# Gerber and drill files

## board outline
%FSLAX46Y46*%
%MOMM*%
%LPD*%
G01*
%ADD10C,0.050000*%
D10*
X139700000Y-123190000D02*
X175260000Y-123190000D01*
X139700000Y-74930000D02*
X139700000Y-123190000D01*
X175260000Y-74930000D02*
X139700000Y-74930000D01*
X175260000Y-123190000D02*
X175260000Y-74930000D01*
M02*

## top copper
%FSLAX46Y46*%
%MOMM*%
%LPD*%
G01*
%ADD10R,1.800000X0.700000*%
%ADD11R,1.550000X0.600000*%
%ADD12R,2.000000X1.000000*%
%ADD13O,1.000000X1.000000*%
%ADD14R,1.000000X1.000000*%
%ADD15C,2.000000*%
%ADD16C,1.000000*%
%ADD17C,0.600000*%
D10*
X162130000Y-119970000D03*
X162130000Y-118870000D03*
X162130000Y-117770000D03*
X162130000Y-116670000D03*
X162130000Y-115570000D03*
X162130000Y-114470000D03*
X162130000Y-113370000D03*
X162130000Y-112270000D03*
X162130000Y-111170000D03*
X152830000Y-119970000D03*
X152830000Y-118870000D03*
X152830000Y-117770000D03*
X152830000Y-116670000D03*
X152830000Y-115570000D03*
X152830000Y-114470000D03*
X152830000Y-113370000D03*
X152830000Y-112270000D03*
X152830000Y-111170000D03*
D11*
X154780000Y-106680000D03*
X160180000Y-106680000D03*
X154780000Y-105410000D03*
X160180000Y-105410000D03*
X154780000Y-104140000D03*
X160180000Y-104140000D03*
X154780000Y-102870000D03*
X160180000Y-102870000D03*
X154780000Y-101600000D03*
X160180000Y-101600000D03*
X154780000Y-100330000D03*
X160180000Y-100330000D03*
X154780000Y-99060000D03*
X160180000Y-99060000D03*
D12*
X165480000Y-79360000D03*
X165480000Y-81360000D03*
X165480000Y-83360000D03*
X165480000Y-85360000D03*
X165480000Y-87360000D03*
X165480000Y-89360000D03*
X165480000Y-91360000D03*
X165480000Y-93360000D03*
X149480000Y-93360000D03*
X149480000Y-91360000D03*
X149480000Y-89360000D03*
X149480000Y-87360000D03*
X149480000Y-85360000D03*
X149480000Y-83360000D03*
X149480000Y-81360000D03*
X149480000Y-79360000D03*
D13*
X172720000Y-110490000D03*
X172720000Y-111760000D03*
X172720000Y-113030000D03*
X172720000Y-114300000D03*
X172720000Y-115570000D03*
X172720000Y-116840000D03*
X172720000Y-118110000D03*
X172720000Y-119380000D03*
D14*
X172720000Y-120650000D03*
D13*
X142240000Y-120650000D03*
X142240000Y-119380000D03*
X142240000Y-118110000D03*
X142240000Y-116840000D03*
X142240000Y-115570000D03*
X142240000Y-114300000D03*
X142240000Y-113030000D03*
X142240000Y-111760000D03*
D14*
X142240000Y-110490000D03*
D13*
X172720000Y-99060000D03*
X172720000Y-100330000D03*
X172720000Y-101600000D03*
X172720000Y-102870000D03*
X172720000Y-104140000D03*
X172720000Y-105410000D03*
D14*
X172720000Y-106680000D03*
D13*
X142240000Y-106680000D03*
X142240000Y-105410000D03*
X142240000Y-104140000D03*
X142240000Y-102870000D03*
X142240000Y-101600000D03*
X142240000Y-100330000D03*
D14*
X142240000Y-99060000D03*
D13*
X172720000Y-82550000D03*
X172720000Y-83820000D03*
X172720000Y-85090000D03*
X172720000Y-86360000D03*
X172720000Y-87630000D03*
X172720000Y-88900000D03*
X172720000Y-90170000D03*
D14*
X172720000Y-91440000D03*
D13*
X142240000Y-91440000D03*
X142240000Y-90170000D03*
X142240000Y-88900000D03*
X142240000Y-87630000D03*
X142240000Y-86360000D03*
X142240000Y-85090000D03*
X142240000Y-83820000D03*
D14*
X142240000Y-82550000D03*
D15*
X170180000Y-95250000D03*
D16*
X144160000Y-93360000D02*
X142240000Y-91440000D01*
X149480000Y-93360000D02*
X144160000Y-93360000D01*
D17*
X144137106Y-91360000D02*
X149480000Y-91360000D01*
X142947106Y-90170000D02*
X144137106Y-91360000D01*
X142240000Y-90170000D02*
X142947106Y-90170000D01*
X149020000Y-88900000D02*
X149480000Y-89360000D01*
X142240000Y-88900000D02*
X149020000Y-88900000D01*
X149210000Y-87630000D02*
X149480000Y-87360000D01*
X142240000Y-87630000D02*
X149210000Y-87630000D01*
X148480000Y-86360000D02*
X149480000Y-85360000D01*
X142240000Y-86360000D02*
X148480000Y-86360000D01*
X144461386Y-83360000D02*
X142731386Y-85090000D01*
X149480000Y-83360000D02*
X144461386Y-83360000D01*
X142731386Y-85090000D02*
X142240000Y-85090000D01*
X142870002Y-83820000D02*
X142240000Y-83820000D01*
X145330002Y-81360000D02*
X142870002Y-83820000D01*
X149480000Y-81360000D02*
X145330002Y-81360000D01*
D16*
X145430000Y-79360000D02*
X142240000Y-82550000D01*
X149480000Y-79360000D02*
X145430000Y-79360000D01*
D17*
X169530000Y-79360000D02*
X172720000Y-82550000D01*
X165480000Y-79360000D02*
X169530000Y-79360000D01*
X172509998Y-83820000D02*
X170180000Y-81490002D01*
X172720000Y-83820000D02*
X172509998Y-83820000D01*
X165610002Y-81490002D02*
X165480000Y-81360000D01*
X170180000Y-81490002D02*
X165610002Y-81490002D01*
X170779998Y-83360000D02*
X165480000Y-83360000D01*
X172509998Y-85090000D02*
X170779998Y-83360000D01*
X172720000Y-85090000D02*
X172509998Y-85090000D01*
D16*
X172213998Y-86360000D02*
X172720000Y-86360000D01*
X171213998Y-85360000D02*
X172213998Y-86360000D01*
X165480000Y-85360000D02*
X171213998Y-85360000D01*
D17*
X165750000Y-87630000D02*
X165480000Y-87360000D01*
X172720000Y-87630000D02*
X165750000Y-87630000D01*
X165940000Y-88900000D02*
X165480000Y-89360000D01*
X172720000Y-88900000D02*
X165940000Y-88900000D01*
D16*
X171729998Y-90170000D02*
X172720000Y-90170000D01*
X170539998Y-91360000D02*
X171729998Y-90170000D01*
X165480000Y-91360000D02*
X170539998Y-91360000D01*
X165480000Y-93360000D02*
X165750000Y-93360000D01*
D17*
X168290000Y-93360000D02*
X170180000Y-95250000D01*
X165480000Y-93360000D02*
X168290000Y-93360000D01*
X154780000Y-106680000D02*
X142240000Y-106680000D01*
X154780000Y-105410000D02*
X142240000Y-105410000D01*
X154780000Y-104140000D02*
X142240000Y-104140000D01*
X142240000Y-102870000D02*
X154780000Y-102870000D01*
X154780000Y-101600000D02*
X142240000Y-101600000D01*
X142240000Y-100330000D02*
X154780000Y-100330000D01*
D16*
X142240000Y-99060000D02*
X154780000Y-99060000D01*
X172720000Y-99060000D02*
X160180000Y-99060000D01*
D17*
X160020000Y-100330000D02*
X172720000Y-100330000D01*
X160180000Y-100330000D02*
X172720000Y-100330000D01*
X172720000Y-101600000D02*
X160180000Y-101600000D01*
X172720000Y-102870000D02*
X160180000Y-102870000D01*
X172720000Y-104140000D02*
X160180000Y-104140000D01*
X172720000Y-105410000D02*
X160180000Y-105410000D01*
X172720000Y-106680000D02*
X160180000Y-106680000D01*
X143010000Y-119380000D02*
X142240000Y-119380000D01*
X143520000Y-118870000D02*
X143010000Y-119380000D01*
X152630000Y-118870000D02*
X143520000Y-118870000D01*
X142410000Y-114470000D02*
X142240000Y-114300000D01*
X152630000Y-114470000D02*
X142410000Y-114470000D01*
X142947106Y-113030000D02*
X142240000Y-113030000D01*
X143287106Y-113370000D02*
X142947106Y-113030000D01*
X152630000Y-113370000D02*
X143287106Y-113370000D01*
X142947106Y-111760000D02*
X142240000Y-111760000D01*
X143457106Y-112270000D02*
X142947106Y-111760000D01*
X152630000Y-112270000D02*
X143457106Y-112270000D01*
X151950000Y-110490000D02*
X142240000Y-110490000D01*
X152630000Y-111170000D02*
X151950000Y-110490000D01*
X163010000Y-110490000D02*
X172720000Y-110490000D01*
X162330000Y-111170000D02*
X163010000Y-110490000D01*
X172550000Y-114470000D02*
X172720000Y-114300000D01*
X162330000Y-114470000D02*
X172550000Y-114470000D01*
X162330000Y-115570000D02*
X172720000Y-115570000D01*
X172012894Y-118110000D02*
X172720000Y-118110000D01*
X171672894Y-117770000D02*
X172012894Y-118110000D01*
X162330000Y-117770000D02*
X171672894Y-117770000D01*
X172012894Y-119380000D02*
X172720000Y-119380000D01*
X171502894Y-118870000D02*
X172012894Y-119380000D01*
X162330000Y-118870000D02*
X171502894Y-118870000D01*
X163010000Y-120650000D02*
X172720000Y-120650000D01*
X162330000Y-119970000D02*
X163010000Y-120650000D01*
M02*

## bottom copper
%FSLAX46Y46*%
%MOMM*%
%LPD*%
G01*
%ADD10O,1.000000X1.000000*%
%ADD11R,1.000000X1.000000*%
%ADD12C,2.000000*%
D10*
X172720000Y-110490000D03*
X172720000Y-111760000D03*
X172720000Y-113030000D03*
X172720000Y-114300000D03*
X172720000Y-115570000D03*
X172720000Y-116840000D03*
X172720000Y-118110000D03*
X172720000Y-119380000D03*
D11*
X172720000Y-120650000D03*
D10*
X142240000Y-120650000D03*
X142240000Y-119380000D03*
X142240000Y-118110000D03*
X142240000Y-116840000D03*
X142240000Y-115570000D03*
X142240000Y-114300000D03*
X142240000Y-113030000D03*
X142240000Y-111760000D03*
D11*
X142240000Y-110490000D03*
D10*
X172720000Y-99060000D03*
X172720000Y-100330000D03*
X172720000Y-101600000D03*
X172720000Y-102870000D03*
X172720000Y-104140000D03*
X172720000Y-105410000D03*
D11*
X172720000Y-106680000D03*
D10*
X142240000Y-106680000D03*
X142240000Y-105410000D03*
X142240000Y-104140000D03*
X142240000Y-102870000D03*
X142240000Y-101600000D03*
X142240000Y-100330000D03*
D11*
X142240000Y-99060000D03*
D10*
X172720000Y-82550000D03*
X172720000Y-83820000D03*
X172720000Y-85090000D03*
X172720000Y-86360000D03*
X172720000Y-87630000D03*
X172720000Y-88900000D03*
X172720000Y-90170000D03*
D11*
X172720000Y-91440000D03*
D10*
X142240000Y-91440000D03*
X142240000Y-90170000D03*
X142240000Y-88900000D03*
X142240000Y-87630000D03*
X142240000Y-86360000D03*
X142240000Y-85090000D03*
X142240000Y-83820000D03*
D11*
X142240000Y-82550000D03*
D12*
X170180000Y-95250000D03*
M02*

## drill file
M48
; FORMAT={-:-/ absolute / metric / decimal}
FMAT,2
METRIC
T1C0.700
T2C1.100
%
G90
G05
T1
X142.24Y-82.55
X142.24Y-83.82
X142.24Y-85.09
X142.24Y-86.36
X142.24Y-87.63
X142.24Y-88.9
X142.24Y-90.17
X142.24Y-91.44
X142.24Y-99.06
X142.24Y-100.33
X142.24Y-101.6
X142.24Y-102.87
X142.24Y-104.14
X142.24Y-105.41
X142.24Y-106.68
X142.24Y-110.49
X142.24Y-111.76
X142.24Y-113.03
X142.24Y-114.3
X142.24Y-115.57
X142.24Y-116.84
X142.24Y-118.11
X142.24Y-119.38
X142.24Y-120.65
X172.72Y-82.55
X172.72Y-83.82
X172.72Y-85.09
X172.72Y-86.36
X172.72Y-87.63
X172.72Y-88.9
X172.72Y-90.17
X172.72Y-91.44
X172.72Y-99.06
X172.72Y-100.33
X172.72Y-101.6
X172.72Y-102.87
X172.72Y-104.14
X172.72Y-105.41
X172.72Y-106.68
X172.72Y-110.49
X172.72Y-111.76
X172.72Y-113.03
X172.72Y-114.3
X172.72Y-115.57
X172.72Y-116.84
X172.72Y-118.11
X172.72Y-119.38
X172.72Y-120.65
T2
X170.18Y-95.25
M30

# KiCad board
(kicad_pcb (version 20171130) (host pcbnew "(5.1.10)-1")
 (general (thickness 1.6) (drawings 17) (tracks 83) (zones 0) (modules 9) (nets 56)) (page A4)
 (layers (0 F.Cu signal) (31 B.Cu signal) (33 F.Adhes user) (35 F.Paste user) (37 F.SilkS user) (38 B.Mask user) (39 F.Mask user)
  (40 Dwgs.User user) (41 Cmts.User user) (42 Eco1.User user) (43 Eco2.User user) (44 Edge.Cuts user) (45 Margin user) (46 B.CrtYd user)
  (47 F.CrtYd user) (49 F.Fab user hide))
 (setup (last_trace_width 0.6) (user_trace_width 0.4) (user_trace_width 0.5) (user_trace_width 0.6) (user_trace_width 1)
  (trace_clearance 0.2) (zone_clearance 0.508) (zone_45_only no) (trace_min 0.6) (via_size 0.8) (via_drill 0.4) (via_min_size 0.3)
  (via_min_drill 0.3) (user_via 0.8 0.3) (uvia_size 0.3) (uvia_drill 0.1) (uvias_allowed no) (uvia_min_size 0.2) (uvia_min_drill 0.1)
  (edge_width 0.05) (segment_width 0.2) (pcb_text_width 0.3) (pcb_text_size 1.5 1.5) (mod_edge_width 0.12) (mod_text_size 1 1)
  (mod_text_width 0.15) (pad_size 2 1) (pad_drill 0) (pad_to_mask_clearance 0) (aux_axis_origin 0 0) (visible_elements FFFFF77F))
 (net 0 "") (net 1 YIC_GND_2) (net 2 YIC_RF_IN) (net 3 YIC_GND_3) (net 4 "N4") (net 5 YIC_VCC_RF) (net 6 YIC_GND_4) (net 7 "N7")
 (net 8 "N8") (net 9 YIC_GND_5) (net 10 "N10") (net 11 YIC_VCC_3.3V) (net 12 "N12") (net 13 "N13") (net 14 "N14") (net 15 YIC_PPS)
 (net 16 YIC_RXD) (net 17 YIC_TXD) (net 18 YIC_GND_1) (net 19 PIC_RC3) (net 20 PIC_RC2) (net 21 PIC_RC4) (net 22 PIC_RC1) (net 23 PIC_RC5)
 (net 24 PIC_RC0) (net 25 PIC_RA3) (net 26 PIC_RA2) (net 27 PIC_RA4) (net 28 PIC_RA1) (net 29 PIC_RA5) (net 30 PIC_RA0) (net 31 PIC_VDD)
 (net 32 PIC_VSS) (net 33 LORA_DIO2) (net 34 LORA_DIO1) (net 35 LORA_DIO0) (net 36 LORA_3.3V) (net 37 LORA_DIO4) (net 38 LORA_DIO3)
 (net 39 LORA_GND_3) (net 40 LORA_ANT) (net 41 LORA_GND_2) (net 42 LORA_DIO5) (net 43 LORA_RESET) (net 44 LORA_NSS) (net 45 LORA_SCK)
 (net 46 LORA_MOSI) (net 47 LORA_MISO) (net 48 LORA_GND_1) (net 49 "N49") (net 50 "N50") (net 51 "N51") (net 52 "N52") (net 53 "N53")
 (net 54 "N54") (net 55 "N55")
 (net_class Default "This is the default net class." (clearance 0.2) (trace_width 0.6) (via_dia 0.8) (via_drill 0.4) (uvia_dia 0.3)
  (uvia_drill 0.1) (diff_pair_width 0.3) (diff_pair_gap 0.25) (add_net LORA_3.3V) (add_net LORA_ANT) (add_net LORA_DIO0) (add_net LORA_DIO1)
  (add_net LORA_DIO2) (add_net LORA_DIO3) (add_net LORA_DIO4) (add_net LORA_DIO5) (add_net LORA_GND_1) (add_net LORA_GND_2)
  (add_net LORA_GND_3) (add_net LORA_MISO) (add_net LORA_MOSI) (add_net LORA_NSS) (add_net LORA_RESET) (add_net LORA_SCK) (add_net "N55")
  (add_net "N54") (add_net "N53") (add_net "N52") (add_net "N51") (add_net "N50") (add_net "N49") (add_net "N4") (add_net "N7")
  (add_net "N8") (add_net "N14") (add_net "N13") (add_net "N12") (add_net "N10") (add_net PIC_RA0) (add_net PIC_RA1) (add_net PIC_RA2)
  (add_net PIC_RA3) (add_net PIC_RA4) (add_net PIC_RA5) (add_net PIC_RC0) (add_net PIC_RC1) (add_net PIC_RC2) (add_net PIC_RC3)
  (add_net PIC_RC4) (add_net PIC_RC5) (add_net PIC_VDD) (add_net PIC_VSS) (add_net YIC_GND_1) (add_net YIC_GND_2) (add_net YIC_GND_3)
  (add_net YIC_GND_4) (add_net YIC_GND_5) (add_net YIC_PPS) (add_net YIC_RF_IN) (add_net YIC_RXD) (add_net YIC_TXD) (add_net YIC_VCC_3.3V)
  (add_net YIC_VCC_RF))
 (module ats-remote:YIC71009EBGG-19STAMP (layer F.Cu) (at 157.48 115.57 270)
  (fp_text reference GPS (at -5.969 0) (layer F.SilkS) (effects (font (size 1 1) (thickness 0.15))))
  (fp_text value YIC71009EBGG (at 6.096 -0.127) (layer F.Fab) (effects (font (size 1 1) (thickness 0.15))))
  (pad 10 smd rect (at 4.4 -4.85 270) (size 0.7 1.8) (drill (offset 0 0.2)) (layers F.Cu F.Paste F.Mask) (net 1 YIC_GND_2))
  (pad 11 smd rect (at 3.3 -4.85 270) (size 0.7 1.8) (drill (offset 0 0.2)) (layers F.Cu F.Paste F.Mask) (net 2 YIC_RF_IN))
  (pad 12 smd rect (at 2.2 -4.85 270) (size 0.7 1.8) (drill (offset 0 0.2)) (layers F.Cu F.Paste F.Mask) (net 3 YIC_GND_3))
  (pad 13 smd rect (at 1.1 -4.85 270) (size 0.7 1.8) (drill (offset 0 0.2)) (layers F.Cu F.Paste F.Mask) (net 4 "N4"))
  (pad 14 smd rect (at 0 -4.85 270) (size 0.7 1.8) (drill (offset 0 0.2)) (layers F.Cu F.Paste F.Mask) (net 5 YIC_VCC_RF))
  (pad 15 smd rect (at -1.1 -4.85 270) (size 0.7 1.8) (drill (offset 0 0.2)) (layers F.Cu F.Paste F.Mask) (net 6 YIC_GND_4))
  (pad 16 smd rect (at -2.2 -4.85 270) (size 0.7 1.8) (drill (offset 0 0.2)) (layers F.Cu F.Paste F.Mask) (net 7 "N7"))
  (pad 17 smd rect (at -3.3 -4.85 270) (size 0.7 1.8) (drill (offset 0 0.2)) (layers F.Cu F.Paste F.Mask) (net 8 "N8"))
  (pad 18 smd rect (at -4.4 -4.85 270) (size 0.7 1.8) (drill (offset 0 0.2)) (layers F.Cu F.Paste F.Mask) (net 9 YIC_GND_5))
  (pad 9 smd rect (at 4.4 4.85 270) (size 0.7 1.8) (drill (offset 0 -0.2)) (layers F.Cu F.Paste F.Mask) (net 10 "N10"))
  (pad 8 smd rect (at 3.3 4.85 270) (size 0.7 1.8) (drill (offset 0 -0.2)) (layers F.Cu F.Paste F.Mask) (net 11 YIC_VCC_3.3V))
  (pad 7 smd rect (at 2.2 4.85 270) (size 0.7 1.8) (drill (offset 0 -0.2)) (layers F.Cu F.Paste F.Mask) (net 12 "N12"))
  (pad 6 smd rect (at 1.1 4.85 270) (size 0.7 1.8) (drill (offset 0 -0.2)) (layers F.Cu F.Paste F.Mask) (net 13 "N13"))
  (pad 5 smd rect (at 0 4.85 270) (size 0.7 1.8) (drill (offset 0 -0.2)) (layers F.Cu F.Paste F.Mask) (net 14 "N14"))
  (pad 4 smd rect (at -1.1 4.85 270) (size 0.7 1.8) (drill (offset 0 -0.2)) (layers F.Cu F.Paste F.Mask) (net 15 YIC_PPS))
  (pad 3 smd rect (at -2.2 4.85 270) (size 0.7 1.8) (drill (offset 0 -0.2)) (layers F.Cu F.Paste F.Mask) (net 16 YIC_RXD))
  (pad 2 smd rect (at -3.3 4.85 270) (size 0.7 1.8) (drill (offset 0 -0.2)) (layers F.Cu F.Paste F.Mask) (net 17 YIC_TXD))
  (pad 1 smd rect (at -4.4 4.85 270) (size 0.7 1.8) (drill (offset 0 -0.2)) (layers F.Cu F.Paste F.Mask) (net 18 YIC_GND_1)))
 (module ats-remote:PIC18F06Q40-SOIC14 (layer F.Cu) (at 157.48 102.87 270)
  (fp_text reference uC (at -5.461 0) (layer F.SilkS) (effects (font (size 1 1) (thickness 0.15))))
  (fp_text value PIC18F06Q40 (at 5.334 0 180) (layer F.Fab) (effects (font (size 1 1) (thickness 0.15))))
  (pad 7 smd rect (at 3.81 2.7 270) (size 0.6 1.55) (layers F.Cu F.Paste F.Mask) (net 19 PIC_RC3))
  (pad 8 smd rect (at 3.81 -2.7 270) (size 0.6 1.55) (layers F.Cu F.Paste F.Mask) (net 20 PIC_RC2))
  (pad 6 smd rect (at 2.54 2.7 270) (size 0.6 1.55) (layers F.Cu F.Paste F.Mask) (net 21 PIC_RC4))
  (pad 9 smd rect (at 2.54 -2.7 270) (size 0.6 1.55) (layers F.Cu F.Paste F.Mask) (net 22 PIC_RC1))
  (pad 5 smd rect (at 1.27 2.7 270) (size 0.6 1.55) (layers F.Cu F.Paste F.Mask) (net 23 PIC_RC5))
  (pad 10 smd rect (at 1.27 -2.7 270) (size 0.6 1.55) (layers F.Cu F.Paste F.Mask) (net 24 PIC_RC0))
  (pad 4 smd rect (at 0 2.7 270) (size 0.6 1.55) (layers F.Cu F.Paste F.Mask) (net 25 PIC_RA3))
  (pad 11 smd rect (at 0 -2.7 270) (size 0.6 1.55) (layers F.Cu F.Paste F.Mask) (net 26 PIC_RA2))
  (pad 3 smd rect (at -1.27 2.7 270) (size 0.6 1.55) (layers F.Cu F.Paste F.Mask) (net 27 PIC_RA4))
  (pad 12 smd rect (at -1.27 -2.7 270) (size 0.6 1.55) (layers F.Cu F.Paste F.Mask) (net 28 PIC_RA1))
  (pad 2 smd rect (at -2.54 2.7 270) (size 0.6 1.55) (layers F.Cu F.Paste F.Mask) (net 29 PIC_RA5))
  (pad 13 smd rect (at -2.54 -2.7 270) (size 0.6 1.55) (layers F.Cu F.Paste F.Mask) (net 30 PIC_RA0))
  (pad 1 smd rect (at -3.81 2.7 270) (size 0.6 1.55) (layers F.Cu F.Paste F.Mask) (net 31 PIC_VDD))
  (pad 14 smd rect (at -3.81 -2.7 270) (size 0.6 1.55) (layers F.Cu F.Paste F.Mask) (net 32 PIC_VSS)))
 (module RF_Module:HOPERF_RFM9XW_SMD (layer F.Cu) (at 157.48 86.36)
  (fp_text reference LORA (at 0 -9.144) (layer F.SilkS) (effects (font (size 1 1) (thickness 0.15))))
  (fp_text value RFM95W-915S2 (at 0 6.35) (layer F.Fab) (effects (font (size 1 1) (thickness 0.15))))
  (pad 16 smd rect (at 8 -7) (size 2 1) (layers F.Cu F.Paste F.Mask) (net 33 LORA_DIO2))
  (pad 15 smd rect (at 8 -5) (size 2 1) (layers F.Cu F.Paste F.Mask) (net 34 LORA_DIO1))
  (pad 14 smd rect (at 8 -3) (size 2 1) (layers F.Cu F.Paste F.Mask) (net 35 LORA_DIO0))
  (pad 13 smd rect (at 8 -1) (size 2 1) (layers F.Cu F.Paste F.Mask) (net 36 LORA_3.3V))
  (pad 12 smd rect (at 8 1) (size 2 1) (layers F.Cu F.Paste F.Mask) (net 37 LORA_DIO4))
  (pad 11 smd rect (at 8 3) (size 2 1) (layers F.Cu F.Paste F.Mask) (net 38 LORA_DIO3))
  (pad 10 smd rect (at 8 5) (size 2 1) (layers F.Cu F.Paste F.Mask) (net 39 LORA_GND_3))
  (pad 9 smd rect (at 8 7) (size 2 1) (layers F.Cu F.Paste F.Mask) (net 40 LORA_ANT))
  (pad 8 smd rect (at -8 7) (size 2 1) (layers F.Cu F.Paste F.Mask) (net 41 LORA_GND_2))
  (pad 7 smd rect (at -8 5) (size 2 1) (layers F.Cu F.Paste F.Mask) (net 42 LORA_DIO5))
  (pad 6 smd rect (at -8 3) (size 2 1) (layers F.Cu F.Paste F.Mask) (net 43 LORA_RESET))
  (pad 5 smd rect (at -8 1) (size 2 1) (layers F.Cu F.Paste F.Mask) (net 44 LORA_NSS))
  (pad 4 smd rect (at -8 -1) (size 2 1) (layers F.Cu F.Paste F.Mask) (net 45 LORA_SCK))
  (pad 3 smd rect (at -8 -3) (size 2 1) (layers F.Cu F.Paste F.Mask) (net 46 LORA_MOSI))
  (pad 2 smd rect (at -8 -5) (size 2 1) (layers F.Cu F.Paste F.Mask) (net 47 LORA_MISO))
  (pad 1 smd rect (at -8 -7) (size 2 1) (layers F.Cu F.Paste F.Mask) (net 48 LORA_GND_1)))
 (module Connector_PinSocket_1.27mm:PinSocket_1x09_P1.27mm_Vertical (layer F.Cu) (at 172.72 120.65 180)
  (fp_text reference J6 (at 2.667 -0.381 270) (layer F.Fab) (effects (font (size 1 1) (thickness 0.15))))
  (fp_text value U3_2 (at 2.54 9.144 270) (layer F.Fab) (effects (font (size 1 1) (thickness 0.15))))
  (pad 9 thru_hole oval (at 0 10.16 180) (size 1 1) (drill 0.7) (layers *.Cu *.Mask) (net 9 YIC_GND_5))
  (pad 8 thru_hole oval (at 0 8.89 180) (size 1 1) (drill 0.7) (layers *.Cu *.Mask) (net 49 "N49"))
  (pad 7 thru_hole oval (at 0 7.62 180) (size 1 1) (drill 0.7) (layers *.Cu *.Mask) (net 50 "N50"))
  (pad 6 thru_hole oval (at 0 6.35 180) (size 1 1) (drill 0.7) (layers *.Cu *.Mask) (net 6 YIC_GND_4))
  (pad 5 thru_hole oval (at 0 5.08 180) (size 1 1) (drill 0.7) (layers *.Cu *.Mask) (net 5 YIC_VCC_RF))
  (pad 4 thru_hole oval (at 0 3.81 180) (size 1 1) (drill 0.7) (layers *.Cu *.Mask) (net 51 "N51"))
  (pad 3 thru_hole oval (at 0 2.54 180) (size 1 1) (drill 0.7) (layers *.Cu *.Mask) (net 3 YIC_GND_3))
  (pad 2 thru_hole oval (at 0 1.27 180) (size 1 1) (drill 0.7) (layers *.Cu *.Mask) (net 2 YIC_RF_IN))
  (pad 1 thru_hole rect (at 0 0 180) (size 1 1) (drill 0.7) (layers *.Cu *.Mask) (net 1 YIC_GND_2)))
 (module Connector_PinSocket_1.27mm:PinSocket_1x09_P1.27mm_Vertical (layer F.Cu) (at 142.24 110.49)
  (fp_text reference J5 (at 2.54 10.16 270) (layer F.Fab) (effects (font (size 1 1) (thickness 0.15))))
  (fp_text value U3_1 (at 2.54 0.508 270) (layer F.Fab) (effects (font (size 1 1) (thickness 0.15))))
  (pad 9 thru_hole oval (at 0 10.16) (size 1 1) (drill 0.7) (layers *.Cu *.Mask) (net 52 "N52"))
  (pad 8 thru_hole oval (at 0 8.89) (size 1 1) (drill 0.7) (layers *.Cu *.Mask) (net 11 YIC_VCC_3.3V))
  (pad 7 thru_hole oval (at 0 7.62) (size 1 1) (drill 0.7) (layers *.Cu *.Mask) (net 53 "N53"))
  (pad 6 thru_hole oval (at 0 6.35) (size 1 1) (drill 0.7) (layers *.Cu *.Mask) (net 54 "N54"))
  (pad 5 thru_hole oval (at 0 5.08) (size 1 1) (drill 0.7) (layers *.Cu *.Mask) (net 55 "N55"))
  (pad 4 thru_hole oval (at 0 3.81) (size 1 1) (drill 0.7) (layers *.Cu *.Mask) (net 15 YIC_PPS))
  (pad 3 thru_hole oval (at 0 2.54) (size 1 1) (drill 0.7) (layers *.Cu *.Mask) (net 16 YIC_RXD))
  (pad 2 thru_hole oval (at 0 1.27) (size 1 1) (drill 0.7) (layers *.Cu *.Mask) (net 17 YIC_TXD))
  (pad 1 thru_hole rect (at 0 0) (size 1 1) (drill 0.7) (layers *.Cu *.Mask) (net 18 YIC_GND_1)))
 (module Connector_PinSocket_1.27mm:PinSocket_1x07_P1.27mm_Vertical (layer F.Cu) (at 172.72 106.68 180)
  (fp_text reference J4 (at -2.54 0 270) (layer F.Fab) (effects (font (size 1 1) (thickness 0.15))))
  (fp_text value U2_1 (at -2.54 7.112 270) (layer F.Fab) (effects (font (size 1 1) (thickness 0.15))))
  (pad 7 thru_hole oval (at 0 7.62 180) (size 1 1) (drill 0.7) (layers *.Cu *.Mask) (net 32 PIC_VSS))
  (pad 6 thru_hole oval (at 0 6.35 180) (size 1 1) (drill 0.7) (layers *.Cu *.Mask) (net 30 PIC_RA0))
  (pad 5 thru_hole oval (at 0 5.08 180) (size 1 1) (drill 0.7) (layers *.Cu *.Mask) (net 28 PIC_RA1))
  (pad 4 thru_hole oval (at 0 3.81 180) (size 1 1) (drill 0.7) (layers *.Cu *.Mask) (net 26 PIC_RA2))
  (pad 3 thru_hole oval (at 0 2.54 180) (size 1 1) (drill 0.7) (layers *.Cu *.Mask) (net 24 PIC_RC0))
  (pad 2 thru_hole oval (at 0 1.27 180) (size 1 1) (drill 0.7) (layers *.Cu *.Mask) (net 22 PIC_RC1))
  (pad 1 thru_hole rect (at 0 0 180) (size 1 1) (drill 0.7) (layers *.Cu *.Mask) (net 20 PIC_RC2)))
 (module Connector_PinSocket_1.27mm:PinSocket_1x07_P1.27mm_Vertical (layer F.Cu) (at 142.24 99.06)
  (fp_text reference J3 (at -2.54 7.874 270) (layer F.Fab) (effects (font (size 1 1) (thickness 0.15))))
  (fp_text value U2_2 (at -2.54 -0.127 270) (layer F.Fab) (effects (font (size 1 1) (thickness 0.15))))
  (pad 7 thru_hole oval (at 0 7.62) (size 1 1) (drill 0.7) (layers *.Cu *.Mask) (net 19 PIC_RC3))
  (pad 6 thru_hole oval (at 0 6.35) (size 1 1) (drill 0.7) (layers *.Cu *.Mask) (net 21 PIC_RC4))
  (pad 5 thru_hole oval (at 0 5.08) (size 1 1) (drill 0.7) (layers *.Cu *.Mask) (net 23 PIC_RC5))
  (pad 4 thru_hole oval (at 0 3.81) (size 1 1) (drill 0.7) (layers *.Cu *.Mask) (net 25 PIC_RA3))
  (pad 3 thru_hole oval (at 0 2.54) (size 1 1) (drill 0.7) (layers *.Cu *.Mask) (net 27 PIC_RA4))
  (pad 2 thru_hole oval (at 0 1.27) (size 1 1) (drill 0.7) (layers *.Cu *.Mask) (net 29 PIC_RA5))
  (pad 1 thru_hole rect (at 0 0) (size 1 1) (drill 0.7) (layers *.Cu *.Mask) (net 31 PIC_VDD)))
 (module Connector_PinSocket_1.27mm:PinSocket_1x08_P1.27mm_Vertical (layer F.Cu) (at 172.72 91.44 180)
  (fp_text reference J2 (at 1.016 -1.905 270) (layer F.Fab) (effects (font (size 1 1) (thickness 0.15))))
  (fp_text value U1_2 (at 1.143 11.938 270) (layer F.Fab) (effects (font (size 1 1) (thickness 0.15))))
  (pad 8 thru_hole oval (at 0 8.89 180) (size 1 1) (drill 0.7) (layers *.Cu *.Mask) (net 33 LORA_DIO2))
  (pad 7 thru_hole oval (at 0 7.62 180) (size 1 1) (drill 0.7) (layers *.Cu *.Mask) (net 34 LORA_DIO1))
  (pad 6 thru_hole oval (at 0 6.35 180) (size 1 1) (drill 0.7) (layers *.Cu *.Mask) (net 35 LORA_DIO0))
  (pad 5 thru_hole oval (at 0 5.08 180) (size 1 1) (drill 0.7) (layers *.Cu *.Mask) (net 36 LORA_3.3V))
  (pad 4 thru_hole oval (at 0 3.81 180) (size 1 1) (drill 0.7) (layers *.Cu *.Mask) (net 37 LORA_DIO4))
  (pad 3 thru_hole oval (at 0 2.54 180) (size 1 1) (drill 0.7) (layers *.Cu *.Mask) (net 38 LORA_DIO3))
  (pad 2 thru_hole oval (at 0 1.27 180) (size 1 1) (drill 0.7) (layers *.Cu *.Mask) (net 39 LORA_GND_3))
  (pad 1 thru_hole rect (at 0 0 180) (size 1 1) (drill 0.7) (layers *.Cu *.Mask) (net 40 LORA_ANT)))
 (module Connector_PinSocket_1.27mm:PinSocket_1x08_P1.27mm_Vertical (layer F.Cu) (at 142.24 82.55)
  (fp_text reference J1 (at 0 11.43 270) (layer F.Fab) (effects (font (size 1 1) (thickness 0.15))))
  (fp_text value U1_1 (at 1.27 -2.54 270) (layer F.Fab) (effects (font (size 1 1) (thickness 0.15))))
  (pad 8 thru_hole oval (at 0 8.89) (size 1 1) (drill 0.7) (layers *.Cu *.Mask) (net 41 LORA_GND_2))
  (pad 7 thru_hole oval (at 0 7.62) (size 1 1) (drill 0.7) (layers *.Cu *.Mask) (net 42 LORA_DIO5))
  (pad 6 thru_hole oval (at 0 6.35) (size 1 1) (drill 0.7) (layers *.Cu *.Mask) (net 43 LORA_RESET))
  (pad 5 thru_hole oval (at 0 5.08) (size 1 1) (drill 0.7) (layers *.Cu *.Mask) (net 44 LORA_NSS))
  (pad 4 thru_hole oval (at 0 3.81) (size 1 1) (drill 0.7) (layers *.Cu *.Mask) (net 45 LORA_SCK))
  (pad 3 thru_hole oval (at 0 2.54) (size 1 1) (drill 0.7) (layers *.Cu *.Mask) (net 46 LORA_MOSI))
  (pad 2 thru_hole oval (at 0 1.27) (size 1 1) (drill 0.7) (layers *.Cu *.Mask) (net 47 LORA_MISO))
  (pad 1 thru_hole rect (at 0 0) (size 1 1) (drill 0.7) (layers *.Cu *.Mask) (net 48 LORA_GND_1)))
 (gr_line (start 139.7 123.19) (end 175.26 123.19) (layer Edge.Cuts) (width 0.05))
 (gr_line (start 139.7 74.93) (end 139.7 123.19) (layer Edge.Cuts) (width 0.05))
 (gr_line (start 175.26 74.93) (end 139.7 74.93) (layer Edge.Cuts) (width 0.05))
 (gr_line (start 175.26 123.19) (end 175.26 74.93) (layer Edge.Cuts) (width 0.05))
 (segment (start 144.16 93.36) (end 142.24 91.44) (width 1) (layer F.Cu) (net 41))
 (segment (start 149.48 93.36) (end 144.16 93.36) (width 1) (layer F.Cu) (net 41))
 (segment (start 144.137106 91.36) (end 149.48 91.36) (width 0.6) (layer F.Cu) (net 42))
 (segment (start 142.947106 90.17) (end 144.137106 91.36) (width 0.6) (layer F.Cu) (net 42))
 (segment (start 142.24 90.17) (end 142.947106 90.17) (width 0.6) (layer F.Cu) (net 42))
 (segment (start 149.02 88.9) (end 149.48 89.36) (width 0.6) (layer F.Cu) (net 43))
 (segment (start 142.24 88.9) (end 149.02 88.9) (width 0.6) (layer F.Cu) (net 43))
 (via (at 170.18 95.25) (size 2) (drill 1.1) (layers F.Cu B.Cu) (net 40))
 (segment (start 149.21 87.63) (end 149.48 87.36) (width 0.6) (layer F.Cu) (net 44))
 (segment (start 142.24 87.63) (end 149.21 87.63) (width 0.6) (layer F.Cu) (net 44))
 (segment (start 148.48 86.36) (end 149.48 85.36) (width 0.6) (layer F.Cu) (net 45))
 (segment (start 142.24 86.36) (end 148.48 86.36) (width 0.6) (layer F.Cu) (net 45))
 (segment (start 144.461386 83.36) (end 142.731386 85.09) (width 0.6) (layer F.Cu) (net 46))
 (segment (start 149.48 83.36) (end 144.461386 83.36) (width 0.6) (layer F.Cu) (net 46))
 (segment (start 142.731386 85.09) (end 142.24 85.09) (width 0.6) (layer F.Cu) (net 46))
 (segment (start 142.870002 83.82) (end 142.24 83.82) (width 0.6) (layer F.Cu) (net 47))
 (segment (start 145.330002 81.36) (end 142.870002 83.82) (width 0.6) (layer F.Cu) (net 47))
 (segment (start 149.48 81.36) (end 145.330002 81.36) (width 0.6) (layer F.Cu) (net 47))
 (segment (start 145.43 79.36) (end 142.24 82.55) (width 1) (layer F.Cu) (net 48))
 (segment (start 149.48 79.36) (end 145.43 79.36) (width 1) (layer F.Cu) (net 48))
 (segment (start 169.53 79.36) (end 172.72 82.55) (width 0.6) (layer F.Cu) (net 33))
 (segment (start 165.48 79.36) (end 169.53 79.36) (width 0.6) (layer F.Cu) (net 33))
 (segment (start 172.509998 83.82) (end 170.18 81.490002) (width 0.6) (layer F.Cu) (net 34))
 (segment (start 172.72 83.82) (end 172.509998 83.82) (width 0.6) (layer F.Cu) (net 34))
 (segment (start 165.610002 81.490002) (end 165.48 81.36) (width 0.6) (layer F.Cu) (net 34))
 (segment (start 170.18 81.490002) (end 165.610002 81.490002) (width 0.6) (layer F.Cu) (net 34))
 (segment (start 170.779998 83.36) (end 165.48 83.36) (width 0.6) (layer F.Cu) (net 35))
 (segment (start 172.509998 85.09) (end 170.779998 83.36) (width 0.6) (layer F.Cu) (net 35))
 (segment (start 172.72 85.09) (end 172.509998 85.09) (width 0.6) (layer F.Cu) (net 35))
 (segment (start 172.213998 86.36) (end 172.72 86.36) (width 1) (layer F.Cu) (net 36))
 (segment (start 171.213998 85.36) (end 172.213998 86.36) (width 1) (layer F.Cu) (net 36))
 (segment (start 165.48 85.36) (end 171.213998 85.36) (width 1) (layer F.Cu) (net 36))
 (segment (start 165.75 87.63) (end 165.48 87.36) (width 0.6) (layer F.Cu) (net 37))
 (segment (start 172.72 87.63) (end 165.75 87.63) (width 0.6) (layer F.Cu) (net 37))
 (segment (start 165.94 88.9) (end 165.48 89.36) (width 0.6) (layer F.Cu) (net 38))
 (segment (start 172.72 88.9) (end 165.94 88.9) (width 0.6) (layer F.Cu) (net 38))
 (segment (start 171.729998 90.17) (end 172.72 90.17) (width 1) (layer F.Cu) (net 39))
 (segment (start 170.539998 91.36) (end 171.729998 90.17) (width 1) (layer F.Cu) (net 39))
 (segment (start 165.48 91.36) (end 170.539998 91.36) (width 1) (layer F.Cu) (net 39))
 (segment (start 165.48 93.36) (end 165.75 93.36) (width 1) (layer F.Cu) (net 40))
 (segment (start 168.29 93.36) (end 170.18 95.25) (width 0.6) (layer F.Cu) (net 40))
 (segment (start 165.48 93.36) (end 168.29 93.36) (width 0.6) (layer F.Cu) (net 40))
 (segment (start 154.78 106.68) (end 142.24 106.68) (width 0.6) (layer F.Cu) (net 19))
 (segment (start 154.78 105.41) (end 142.24 105.41) (width 0.6) (layer F.Cu) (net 21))
 (segment (start 154.78 104.14) (end 142.24 104.14) (width 0.6) (layer F.Cu) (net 23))
 (segment (start 142.24 102.87) (end 154.78 102.87) (width 0.6) (layer F.Cu) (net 25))
 (segment (start 154.78 101.6) (end 142.24 101.6) (width 0.6) (layer F.Cu) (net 27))
 (segment (start 142.24 100.33) (end 154.78 100.33) (width 0.6) (layer F.Cu) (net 29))
 (segment (start 142.24 99.06) (end 154.78 99.06) (width 1) (layer F.Cu) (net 31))
 (segment (start 172.72 99.06) (end 160.18 99.06) (width 1) (layer F.Cu) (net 32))
 (segment (start 160.02 100.33) (end 172.72 100.33) (width 0.6) (layer F.Cu) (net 30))
 (segment (start 160.18 100.33) (end 172.72 100.33) (width 0.6) (layer F.Cu) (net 30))
 (segment (start 172.72 101.6) (end 160.18 101.6) (width 0.6) (layer F.Cu) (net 28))
 (segment (start 172.72 102.87) (end 160.18 102.87) (width 0.6) (layer F.Cu) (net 26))
 (segment (start 172.72 104.14) (end 160.18 104.14) (width 0.6) (layer F.Cu) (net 24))
 (segment (start 172.72 105.41) (end 160.18 105.41) (width 0.6) (layer F.Cu) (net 22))
 (segment (start 172.72 106.68) (end 160.18 106.68) (width 0.6) (layer F.Cu) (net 20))
 (segment (start 143.01 119.38) (end 142.24 119.38) (width 0.6) (layer F.Cu) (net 11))
 (segment (start 143.52 118.87) (end 143.01 119.38) (width 0.6) (layer F.Cu) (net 11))
 (segment (start 152.63 118.87) (end 143.52 118.87) (width 0.6) (layer F.Cu) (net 11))
 (segment (start 142.41 114.47) (end 142.24 114.3) (width 0.6) (layer F.Cu) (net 15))
 (segment (start 152.63 114.47) (end 142.41 114.47) (width 0.6) (layer F.Cu) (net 15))
 (segment (start 142.947106 113.03) (end 142.24 113.03) (width 0.6) (layer F.Cu) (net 16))
 (segment (start 143.287106 113.37) (end 142.947106 113.03) (width 0.6) (layer F.Cu) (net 16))
 (segment (start 152.63 113.37) (end 143.287106 113.37) (width 0.6) (layer F.Cu) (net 16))
 (segment (start 142.947106 111.76) (end 142.24 111.76) (width 0.6) (layer F.Cu) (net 17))
 (segment (start 143.457106 112.27) (end 142.947106 111.76) (width 0.6) (layer F.Cu) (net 17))
 (segment (start 152.63 112.27) (end 143.457106 112.27) (width 0.6) (layer F.Cu) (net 17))
 (segment (start 151.95 110.49) (end 142.24 110.49) (width 0.6) (layer F.Cu) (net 18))
 (segment (start 152.63 111.17) (end 151.95 110.49) (width 0.6) (layer F.Cu) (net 18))
 (segment (start 163.01 110.49) (end 172.72 110.49) (width 0.6) (layer F.Cu) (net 9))
 (segment (start 162.33 111.17) (end 163.01 110.49) (width 0.6) (layer F.Cu) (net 9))
 (segment (start 172.55 114.47) (end 172.72 114.3) (width 0.6) (layer F.Cu) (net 6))
 (segment (start 162.33 114.47) (end 172.55 114.47) (width 0.6) (layer F.Cu) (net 6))
 (segment (start 162.33 115.57) (end 172.72 115.57) (width 0.6) (layer F.Cu) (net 5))
 (segment (start 172.012894 118.11) (end 172.72 118.11) (width 0.6) (layer F.Cu) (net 3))
 (segment (start 171.672894 117.77) (end 172.012894 118.11) (width 0.6) (layer F.Cu) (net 3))
 (segment (start 162.33 117.77) (end 171.672894 117.77) (width 0.6) (layer F.Cu) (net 3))
 (segment (start 172.012894 119.38) (end 172.72 119.38) (width 0.6) (layer F.Cu) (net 2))
 (segment (start 171.502894 118.87) (end 172.012894 119.38) (width 0.6) (layer F.Cu) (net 2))
 (segment (start 162.33 118.87) (end 171.502894 118.87) (width 0.6) (layer F.Cu) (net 2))
 (segment (start 163.01 120.65) (end 172.72 120.65) (width 0.6) (layer F.Cu) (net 1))
 (segment (start 162.33 119.97) (end 163.01 120.65) (width 0.6) (layer F.Cu) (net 1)))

